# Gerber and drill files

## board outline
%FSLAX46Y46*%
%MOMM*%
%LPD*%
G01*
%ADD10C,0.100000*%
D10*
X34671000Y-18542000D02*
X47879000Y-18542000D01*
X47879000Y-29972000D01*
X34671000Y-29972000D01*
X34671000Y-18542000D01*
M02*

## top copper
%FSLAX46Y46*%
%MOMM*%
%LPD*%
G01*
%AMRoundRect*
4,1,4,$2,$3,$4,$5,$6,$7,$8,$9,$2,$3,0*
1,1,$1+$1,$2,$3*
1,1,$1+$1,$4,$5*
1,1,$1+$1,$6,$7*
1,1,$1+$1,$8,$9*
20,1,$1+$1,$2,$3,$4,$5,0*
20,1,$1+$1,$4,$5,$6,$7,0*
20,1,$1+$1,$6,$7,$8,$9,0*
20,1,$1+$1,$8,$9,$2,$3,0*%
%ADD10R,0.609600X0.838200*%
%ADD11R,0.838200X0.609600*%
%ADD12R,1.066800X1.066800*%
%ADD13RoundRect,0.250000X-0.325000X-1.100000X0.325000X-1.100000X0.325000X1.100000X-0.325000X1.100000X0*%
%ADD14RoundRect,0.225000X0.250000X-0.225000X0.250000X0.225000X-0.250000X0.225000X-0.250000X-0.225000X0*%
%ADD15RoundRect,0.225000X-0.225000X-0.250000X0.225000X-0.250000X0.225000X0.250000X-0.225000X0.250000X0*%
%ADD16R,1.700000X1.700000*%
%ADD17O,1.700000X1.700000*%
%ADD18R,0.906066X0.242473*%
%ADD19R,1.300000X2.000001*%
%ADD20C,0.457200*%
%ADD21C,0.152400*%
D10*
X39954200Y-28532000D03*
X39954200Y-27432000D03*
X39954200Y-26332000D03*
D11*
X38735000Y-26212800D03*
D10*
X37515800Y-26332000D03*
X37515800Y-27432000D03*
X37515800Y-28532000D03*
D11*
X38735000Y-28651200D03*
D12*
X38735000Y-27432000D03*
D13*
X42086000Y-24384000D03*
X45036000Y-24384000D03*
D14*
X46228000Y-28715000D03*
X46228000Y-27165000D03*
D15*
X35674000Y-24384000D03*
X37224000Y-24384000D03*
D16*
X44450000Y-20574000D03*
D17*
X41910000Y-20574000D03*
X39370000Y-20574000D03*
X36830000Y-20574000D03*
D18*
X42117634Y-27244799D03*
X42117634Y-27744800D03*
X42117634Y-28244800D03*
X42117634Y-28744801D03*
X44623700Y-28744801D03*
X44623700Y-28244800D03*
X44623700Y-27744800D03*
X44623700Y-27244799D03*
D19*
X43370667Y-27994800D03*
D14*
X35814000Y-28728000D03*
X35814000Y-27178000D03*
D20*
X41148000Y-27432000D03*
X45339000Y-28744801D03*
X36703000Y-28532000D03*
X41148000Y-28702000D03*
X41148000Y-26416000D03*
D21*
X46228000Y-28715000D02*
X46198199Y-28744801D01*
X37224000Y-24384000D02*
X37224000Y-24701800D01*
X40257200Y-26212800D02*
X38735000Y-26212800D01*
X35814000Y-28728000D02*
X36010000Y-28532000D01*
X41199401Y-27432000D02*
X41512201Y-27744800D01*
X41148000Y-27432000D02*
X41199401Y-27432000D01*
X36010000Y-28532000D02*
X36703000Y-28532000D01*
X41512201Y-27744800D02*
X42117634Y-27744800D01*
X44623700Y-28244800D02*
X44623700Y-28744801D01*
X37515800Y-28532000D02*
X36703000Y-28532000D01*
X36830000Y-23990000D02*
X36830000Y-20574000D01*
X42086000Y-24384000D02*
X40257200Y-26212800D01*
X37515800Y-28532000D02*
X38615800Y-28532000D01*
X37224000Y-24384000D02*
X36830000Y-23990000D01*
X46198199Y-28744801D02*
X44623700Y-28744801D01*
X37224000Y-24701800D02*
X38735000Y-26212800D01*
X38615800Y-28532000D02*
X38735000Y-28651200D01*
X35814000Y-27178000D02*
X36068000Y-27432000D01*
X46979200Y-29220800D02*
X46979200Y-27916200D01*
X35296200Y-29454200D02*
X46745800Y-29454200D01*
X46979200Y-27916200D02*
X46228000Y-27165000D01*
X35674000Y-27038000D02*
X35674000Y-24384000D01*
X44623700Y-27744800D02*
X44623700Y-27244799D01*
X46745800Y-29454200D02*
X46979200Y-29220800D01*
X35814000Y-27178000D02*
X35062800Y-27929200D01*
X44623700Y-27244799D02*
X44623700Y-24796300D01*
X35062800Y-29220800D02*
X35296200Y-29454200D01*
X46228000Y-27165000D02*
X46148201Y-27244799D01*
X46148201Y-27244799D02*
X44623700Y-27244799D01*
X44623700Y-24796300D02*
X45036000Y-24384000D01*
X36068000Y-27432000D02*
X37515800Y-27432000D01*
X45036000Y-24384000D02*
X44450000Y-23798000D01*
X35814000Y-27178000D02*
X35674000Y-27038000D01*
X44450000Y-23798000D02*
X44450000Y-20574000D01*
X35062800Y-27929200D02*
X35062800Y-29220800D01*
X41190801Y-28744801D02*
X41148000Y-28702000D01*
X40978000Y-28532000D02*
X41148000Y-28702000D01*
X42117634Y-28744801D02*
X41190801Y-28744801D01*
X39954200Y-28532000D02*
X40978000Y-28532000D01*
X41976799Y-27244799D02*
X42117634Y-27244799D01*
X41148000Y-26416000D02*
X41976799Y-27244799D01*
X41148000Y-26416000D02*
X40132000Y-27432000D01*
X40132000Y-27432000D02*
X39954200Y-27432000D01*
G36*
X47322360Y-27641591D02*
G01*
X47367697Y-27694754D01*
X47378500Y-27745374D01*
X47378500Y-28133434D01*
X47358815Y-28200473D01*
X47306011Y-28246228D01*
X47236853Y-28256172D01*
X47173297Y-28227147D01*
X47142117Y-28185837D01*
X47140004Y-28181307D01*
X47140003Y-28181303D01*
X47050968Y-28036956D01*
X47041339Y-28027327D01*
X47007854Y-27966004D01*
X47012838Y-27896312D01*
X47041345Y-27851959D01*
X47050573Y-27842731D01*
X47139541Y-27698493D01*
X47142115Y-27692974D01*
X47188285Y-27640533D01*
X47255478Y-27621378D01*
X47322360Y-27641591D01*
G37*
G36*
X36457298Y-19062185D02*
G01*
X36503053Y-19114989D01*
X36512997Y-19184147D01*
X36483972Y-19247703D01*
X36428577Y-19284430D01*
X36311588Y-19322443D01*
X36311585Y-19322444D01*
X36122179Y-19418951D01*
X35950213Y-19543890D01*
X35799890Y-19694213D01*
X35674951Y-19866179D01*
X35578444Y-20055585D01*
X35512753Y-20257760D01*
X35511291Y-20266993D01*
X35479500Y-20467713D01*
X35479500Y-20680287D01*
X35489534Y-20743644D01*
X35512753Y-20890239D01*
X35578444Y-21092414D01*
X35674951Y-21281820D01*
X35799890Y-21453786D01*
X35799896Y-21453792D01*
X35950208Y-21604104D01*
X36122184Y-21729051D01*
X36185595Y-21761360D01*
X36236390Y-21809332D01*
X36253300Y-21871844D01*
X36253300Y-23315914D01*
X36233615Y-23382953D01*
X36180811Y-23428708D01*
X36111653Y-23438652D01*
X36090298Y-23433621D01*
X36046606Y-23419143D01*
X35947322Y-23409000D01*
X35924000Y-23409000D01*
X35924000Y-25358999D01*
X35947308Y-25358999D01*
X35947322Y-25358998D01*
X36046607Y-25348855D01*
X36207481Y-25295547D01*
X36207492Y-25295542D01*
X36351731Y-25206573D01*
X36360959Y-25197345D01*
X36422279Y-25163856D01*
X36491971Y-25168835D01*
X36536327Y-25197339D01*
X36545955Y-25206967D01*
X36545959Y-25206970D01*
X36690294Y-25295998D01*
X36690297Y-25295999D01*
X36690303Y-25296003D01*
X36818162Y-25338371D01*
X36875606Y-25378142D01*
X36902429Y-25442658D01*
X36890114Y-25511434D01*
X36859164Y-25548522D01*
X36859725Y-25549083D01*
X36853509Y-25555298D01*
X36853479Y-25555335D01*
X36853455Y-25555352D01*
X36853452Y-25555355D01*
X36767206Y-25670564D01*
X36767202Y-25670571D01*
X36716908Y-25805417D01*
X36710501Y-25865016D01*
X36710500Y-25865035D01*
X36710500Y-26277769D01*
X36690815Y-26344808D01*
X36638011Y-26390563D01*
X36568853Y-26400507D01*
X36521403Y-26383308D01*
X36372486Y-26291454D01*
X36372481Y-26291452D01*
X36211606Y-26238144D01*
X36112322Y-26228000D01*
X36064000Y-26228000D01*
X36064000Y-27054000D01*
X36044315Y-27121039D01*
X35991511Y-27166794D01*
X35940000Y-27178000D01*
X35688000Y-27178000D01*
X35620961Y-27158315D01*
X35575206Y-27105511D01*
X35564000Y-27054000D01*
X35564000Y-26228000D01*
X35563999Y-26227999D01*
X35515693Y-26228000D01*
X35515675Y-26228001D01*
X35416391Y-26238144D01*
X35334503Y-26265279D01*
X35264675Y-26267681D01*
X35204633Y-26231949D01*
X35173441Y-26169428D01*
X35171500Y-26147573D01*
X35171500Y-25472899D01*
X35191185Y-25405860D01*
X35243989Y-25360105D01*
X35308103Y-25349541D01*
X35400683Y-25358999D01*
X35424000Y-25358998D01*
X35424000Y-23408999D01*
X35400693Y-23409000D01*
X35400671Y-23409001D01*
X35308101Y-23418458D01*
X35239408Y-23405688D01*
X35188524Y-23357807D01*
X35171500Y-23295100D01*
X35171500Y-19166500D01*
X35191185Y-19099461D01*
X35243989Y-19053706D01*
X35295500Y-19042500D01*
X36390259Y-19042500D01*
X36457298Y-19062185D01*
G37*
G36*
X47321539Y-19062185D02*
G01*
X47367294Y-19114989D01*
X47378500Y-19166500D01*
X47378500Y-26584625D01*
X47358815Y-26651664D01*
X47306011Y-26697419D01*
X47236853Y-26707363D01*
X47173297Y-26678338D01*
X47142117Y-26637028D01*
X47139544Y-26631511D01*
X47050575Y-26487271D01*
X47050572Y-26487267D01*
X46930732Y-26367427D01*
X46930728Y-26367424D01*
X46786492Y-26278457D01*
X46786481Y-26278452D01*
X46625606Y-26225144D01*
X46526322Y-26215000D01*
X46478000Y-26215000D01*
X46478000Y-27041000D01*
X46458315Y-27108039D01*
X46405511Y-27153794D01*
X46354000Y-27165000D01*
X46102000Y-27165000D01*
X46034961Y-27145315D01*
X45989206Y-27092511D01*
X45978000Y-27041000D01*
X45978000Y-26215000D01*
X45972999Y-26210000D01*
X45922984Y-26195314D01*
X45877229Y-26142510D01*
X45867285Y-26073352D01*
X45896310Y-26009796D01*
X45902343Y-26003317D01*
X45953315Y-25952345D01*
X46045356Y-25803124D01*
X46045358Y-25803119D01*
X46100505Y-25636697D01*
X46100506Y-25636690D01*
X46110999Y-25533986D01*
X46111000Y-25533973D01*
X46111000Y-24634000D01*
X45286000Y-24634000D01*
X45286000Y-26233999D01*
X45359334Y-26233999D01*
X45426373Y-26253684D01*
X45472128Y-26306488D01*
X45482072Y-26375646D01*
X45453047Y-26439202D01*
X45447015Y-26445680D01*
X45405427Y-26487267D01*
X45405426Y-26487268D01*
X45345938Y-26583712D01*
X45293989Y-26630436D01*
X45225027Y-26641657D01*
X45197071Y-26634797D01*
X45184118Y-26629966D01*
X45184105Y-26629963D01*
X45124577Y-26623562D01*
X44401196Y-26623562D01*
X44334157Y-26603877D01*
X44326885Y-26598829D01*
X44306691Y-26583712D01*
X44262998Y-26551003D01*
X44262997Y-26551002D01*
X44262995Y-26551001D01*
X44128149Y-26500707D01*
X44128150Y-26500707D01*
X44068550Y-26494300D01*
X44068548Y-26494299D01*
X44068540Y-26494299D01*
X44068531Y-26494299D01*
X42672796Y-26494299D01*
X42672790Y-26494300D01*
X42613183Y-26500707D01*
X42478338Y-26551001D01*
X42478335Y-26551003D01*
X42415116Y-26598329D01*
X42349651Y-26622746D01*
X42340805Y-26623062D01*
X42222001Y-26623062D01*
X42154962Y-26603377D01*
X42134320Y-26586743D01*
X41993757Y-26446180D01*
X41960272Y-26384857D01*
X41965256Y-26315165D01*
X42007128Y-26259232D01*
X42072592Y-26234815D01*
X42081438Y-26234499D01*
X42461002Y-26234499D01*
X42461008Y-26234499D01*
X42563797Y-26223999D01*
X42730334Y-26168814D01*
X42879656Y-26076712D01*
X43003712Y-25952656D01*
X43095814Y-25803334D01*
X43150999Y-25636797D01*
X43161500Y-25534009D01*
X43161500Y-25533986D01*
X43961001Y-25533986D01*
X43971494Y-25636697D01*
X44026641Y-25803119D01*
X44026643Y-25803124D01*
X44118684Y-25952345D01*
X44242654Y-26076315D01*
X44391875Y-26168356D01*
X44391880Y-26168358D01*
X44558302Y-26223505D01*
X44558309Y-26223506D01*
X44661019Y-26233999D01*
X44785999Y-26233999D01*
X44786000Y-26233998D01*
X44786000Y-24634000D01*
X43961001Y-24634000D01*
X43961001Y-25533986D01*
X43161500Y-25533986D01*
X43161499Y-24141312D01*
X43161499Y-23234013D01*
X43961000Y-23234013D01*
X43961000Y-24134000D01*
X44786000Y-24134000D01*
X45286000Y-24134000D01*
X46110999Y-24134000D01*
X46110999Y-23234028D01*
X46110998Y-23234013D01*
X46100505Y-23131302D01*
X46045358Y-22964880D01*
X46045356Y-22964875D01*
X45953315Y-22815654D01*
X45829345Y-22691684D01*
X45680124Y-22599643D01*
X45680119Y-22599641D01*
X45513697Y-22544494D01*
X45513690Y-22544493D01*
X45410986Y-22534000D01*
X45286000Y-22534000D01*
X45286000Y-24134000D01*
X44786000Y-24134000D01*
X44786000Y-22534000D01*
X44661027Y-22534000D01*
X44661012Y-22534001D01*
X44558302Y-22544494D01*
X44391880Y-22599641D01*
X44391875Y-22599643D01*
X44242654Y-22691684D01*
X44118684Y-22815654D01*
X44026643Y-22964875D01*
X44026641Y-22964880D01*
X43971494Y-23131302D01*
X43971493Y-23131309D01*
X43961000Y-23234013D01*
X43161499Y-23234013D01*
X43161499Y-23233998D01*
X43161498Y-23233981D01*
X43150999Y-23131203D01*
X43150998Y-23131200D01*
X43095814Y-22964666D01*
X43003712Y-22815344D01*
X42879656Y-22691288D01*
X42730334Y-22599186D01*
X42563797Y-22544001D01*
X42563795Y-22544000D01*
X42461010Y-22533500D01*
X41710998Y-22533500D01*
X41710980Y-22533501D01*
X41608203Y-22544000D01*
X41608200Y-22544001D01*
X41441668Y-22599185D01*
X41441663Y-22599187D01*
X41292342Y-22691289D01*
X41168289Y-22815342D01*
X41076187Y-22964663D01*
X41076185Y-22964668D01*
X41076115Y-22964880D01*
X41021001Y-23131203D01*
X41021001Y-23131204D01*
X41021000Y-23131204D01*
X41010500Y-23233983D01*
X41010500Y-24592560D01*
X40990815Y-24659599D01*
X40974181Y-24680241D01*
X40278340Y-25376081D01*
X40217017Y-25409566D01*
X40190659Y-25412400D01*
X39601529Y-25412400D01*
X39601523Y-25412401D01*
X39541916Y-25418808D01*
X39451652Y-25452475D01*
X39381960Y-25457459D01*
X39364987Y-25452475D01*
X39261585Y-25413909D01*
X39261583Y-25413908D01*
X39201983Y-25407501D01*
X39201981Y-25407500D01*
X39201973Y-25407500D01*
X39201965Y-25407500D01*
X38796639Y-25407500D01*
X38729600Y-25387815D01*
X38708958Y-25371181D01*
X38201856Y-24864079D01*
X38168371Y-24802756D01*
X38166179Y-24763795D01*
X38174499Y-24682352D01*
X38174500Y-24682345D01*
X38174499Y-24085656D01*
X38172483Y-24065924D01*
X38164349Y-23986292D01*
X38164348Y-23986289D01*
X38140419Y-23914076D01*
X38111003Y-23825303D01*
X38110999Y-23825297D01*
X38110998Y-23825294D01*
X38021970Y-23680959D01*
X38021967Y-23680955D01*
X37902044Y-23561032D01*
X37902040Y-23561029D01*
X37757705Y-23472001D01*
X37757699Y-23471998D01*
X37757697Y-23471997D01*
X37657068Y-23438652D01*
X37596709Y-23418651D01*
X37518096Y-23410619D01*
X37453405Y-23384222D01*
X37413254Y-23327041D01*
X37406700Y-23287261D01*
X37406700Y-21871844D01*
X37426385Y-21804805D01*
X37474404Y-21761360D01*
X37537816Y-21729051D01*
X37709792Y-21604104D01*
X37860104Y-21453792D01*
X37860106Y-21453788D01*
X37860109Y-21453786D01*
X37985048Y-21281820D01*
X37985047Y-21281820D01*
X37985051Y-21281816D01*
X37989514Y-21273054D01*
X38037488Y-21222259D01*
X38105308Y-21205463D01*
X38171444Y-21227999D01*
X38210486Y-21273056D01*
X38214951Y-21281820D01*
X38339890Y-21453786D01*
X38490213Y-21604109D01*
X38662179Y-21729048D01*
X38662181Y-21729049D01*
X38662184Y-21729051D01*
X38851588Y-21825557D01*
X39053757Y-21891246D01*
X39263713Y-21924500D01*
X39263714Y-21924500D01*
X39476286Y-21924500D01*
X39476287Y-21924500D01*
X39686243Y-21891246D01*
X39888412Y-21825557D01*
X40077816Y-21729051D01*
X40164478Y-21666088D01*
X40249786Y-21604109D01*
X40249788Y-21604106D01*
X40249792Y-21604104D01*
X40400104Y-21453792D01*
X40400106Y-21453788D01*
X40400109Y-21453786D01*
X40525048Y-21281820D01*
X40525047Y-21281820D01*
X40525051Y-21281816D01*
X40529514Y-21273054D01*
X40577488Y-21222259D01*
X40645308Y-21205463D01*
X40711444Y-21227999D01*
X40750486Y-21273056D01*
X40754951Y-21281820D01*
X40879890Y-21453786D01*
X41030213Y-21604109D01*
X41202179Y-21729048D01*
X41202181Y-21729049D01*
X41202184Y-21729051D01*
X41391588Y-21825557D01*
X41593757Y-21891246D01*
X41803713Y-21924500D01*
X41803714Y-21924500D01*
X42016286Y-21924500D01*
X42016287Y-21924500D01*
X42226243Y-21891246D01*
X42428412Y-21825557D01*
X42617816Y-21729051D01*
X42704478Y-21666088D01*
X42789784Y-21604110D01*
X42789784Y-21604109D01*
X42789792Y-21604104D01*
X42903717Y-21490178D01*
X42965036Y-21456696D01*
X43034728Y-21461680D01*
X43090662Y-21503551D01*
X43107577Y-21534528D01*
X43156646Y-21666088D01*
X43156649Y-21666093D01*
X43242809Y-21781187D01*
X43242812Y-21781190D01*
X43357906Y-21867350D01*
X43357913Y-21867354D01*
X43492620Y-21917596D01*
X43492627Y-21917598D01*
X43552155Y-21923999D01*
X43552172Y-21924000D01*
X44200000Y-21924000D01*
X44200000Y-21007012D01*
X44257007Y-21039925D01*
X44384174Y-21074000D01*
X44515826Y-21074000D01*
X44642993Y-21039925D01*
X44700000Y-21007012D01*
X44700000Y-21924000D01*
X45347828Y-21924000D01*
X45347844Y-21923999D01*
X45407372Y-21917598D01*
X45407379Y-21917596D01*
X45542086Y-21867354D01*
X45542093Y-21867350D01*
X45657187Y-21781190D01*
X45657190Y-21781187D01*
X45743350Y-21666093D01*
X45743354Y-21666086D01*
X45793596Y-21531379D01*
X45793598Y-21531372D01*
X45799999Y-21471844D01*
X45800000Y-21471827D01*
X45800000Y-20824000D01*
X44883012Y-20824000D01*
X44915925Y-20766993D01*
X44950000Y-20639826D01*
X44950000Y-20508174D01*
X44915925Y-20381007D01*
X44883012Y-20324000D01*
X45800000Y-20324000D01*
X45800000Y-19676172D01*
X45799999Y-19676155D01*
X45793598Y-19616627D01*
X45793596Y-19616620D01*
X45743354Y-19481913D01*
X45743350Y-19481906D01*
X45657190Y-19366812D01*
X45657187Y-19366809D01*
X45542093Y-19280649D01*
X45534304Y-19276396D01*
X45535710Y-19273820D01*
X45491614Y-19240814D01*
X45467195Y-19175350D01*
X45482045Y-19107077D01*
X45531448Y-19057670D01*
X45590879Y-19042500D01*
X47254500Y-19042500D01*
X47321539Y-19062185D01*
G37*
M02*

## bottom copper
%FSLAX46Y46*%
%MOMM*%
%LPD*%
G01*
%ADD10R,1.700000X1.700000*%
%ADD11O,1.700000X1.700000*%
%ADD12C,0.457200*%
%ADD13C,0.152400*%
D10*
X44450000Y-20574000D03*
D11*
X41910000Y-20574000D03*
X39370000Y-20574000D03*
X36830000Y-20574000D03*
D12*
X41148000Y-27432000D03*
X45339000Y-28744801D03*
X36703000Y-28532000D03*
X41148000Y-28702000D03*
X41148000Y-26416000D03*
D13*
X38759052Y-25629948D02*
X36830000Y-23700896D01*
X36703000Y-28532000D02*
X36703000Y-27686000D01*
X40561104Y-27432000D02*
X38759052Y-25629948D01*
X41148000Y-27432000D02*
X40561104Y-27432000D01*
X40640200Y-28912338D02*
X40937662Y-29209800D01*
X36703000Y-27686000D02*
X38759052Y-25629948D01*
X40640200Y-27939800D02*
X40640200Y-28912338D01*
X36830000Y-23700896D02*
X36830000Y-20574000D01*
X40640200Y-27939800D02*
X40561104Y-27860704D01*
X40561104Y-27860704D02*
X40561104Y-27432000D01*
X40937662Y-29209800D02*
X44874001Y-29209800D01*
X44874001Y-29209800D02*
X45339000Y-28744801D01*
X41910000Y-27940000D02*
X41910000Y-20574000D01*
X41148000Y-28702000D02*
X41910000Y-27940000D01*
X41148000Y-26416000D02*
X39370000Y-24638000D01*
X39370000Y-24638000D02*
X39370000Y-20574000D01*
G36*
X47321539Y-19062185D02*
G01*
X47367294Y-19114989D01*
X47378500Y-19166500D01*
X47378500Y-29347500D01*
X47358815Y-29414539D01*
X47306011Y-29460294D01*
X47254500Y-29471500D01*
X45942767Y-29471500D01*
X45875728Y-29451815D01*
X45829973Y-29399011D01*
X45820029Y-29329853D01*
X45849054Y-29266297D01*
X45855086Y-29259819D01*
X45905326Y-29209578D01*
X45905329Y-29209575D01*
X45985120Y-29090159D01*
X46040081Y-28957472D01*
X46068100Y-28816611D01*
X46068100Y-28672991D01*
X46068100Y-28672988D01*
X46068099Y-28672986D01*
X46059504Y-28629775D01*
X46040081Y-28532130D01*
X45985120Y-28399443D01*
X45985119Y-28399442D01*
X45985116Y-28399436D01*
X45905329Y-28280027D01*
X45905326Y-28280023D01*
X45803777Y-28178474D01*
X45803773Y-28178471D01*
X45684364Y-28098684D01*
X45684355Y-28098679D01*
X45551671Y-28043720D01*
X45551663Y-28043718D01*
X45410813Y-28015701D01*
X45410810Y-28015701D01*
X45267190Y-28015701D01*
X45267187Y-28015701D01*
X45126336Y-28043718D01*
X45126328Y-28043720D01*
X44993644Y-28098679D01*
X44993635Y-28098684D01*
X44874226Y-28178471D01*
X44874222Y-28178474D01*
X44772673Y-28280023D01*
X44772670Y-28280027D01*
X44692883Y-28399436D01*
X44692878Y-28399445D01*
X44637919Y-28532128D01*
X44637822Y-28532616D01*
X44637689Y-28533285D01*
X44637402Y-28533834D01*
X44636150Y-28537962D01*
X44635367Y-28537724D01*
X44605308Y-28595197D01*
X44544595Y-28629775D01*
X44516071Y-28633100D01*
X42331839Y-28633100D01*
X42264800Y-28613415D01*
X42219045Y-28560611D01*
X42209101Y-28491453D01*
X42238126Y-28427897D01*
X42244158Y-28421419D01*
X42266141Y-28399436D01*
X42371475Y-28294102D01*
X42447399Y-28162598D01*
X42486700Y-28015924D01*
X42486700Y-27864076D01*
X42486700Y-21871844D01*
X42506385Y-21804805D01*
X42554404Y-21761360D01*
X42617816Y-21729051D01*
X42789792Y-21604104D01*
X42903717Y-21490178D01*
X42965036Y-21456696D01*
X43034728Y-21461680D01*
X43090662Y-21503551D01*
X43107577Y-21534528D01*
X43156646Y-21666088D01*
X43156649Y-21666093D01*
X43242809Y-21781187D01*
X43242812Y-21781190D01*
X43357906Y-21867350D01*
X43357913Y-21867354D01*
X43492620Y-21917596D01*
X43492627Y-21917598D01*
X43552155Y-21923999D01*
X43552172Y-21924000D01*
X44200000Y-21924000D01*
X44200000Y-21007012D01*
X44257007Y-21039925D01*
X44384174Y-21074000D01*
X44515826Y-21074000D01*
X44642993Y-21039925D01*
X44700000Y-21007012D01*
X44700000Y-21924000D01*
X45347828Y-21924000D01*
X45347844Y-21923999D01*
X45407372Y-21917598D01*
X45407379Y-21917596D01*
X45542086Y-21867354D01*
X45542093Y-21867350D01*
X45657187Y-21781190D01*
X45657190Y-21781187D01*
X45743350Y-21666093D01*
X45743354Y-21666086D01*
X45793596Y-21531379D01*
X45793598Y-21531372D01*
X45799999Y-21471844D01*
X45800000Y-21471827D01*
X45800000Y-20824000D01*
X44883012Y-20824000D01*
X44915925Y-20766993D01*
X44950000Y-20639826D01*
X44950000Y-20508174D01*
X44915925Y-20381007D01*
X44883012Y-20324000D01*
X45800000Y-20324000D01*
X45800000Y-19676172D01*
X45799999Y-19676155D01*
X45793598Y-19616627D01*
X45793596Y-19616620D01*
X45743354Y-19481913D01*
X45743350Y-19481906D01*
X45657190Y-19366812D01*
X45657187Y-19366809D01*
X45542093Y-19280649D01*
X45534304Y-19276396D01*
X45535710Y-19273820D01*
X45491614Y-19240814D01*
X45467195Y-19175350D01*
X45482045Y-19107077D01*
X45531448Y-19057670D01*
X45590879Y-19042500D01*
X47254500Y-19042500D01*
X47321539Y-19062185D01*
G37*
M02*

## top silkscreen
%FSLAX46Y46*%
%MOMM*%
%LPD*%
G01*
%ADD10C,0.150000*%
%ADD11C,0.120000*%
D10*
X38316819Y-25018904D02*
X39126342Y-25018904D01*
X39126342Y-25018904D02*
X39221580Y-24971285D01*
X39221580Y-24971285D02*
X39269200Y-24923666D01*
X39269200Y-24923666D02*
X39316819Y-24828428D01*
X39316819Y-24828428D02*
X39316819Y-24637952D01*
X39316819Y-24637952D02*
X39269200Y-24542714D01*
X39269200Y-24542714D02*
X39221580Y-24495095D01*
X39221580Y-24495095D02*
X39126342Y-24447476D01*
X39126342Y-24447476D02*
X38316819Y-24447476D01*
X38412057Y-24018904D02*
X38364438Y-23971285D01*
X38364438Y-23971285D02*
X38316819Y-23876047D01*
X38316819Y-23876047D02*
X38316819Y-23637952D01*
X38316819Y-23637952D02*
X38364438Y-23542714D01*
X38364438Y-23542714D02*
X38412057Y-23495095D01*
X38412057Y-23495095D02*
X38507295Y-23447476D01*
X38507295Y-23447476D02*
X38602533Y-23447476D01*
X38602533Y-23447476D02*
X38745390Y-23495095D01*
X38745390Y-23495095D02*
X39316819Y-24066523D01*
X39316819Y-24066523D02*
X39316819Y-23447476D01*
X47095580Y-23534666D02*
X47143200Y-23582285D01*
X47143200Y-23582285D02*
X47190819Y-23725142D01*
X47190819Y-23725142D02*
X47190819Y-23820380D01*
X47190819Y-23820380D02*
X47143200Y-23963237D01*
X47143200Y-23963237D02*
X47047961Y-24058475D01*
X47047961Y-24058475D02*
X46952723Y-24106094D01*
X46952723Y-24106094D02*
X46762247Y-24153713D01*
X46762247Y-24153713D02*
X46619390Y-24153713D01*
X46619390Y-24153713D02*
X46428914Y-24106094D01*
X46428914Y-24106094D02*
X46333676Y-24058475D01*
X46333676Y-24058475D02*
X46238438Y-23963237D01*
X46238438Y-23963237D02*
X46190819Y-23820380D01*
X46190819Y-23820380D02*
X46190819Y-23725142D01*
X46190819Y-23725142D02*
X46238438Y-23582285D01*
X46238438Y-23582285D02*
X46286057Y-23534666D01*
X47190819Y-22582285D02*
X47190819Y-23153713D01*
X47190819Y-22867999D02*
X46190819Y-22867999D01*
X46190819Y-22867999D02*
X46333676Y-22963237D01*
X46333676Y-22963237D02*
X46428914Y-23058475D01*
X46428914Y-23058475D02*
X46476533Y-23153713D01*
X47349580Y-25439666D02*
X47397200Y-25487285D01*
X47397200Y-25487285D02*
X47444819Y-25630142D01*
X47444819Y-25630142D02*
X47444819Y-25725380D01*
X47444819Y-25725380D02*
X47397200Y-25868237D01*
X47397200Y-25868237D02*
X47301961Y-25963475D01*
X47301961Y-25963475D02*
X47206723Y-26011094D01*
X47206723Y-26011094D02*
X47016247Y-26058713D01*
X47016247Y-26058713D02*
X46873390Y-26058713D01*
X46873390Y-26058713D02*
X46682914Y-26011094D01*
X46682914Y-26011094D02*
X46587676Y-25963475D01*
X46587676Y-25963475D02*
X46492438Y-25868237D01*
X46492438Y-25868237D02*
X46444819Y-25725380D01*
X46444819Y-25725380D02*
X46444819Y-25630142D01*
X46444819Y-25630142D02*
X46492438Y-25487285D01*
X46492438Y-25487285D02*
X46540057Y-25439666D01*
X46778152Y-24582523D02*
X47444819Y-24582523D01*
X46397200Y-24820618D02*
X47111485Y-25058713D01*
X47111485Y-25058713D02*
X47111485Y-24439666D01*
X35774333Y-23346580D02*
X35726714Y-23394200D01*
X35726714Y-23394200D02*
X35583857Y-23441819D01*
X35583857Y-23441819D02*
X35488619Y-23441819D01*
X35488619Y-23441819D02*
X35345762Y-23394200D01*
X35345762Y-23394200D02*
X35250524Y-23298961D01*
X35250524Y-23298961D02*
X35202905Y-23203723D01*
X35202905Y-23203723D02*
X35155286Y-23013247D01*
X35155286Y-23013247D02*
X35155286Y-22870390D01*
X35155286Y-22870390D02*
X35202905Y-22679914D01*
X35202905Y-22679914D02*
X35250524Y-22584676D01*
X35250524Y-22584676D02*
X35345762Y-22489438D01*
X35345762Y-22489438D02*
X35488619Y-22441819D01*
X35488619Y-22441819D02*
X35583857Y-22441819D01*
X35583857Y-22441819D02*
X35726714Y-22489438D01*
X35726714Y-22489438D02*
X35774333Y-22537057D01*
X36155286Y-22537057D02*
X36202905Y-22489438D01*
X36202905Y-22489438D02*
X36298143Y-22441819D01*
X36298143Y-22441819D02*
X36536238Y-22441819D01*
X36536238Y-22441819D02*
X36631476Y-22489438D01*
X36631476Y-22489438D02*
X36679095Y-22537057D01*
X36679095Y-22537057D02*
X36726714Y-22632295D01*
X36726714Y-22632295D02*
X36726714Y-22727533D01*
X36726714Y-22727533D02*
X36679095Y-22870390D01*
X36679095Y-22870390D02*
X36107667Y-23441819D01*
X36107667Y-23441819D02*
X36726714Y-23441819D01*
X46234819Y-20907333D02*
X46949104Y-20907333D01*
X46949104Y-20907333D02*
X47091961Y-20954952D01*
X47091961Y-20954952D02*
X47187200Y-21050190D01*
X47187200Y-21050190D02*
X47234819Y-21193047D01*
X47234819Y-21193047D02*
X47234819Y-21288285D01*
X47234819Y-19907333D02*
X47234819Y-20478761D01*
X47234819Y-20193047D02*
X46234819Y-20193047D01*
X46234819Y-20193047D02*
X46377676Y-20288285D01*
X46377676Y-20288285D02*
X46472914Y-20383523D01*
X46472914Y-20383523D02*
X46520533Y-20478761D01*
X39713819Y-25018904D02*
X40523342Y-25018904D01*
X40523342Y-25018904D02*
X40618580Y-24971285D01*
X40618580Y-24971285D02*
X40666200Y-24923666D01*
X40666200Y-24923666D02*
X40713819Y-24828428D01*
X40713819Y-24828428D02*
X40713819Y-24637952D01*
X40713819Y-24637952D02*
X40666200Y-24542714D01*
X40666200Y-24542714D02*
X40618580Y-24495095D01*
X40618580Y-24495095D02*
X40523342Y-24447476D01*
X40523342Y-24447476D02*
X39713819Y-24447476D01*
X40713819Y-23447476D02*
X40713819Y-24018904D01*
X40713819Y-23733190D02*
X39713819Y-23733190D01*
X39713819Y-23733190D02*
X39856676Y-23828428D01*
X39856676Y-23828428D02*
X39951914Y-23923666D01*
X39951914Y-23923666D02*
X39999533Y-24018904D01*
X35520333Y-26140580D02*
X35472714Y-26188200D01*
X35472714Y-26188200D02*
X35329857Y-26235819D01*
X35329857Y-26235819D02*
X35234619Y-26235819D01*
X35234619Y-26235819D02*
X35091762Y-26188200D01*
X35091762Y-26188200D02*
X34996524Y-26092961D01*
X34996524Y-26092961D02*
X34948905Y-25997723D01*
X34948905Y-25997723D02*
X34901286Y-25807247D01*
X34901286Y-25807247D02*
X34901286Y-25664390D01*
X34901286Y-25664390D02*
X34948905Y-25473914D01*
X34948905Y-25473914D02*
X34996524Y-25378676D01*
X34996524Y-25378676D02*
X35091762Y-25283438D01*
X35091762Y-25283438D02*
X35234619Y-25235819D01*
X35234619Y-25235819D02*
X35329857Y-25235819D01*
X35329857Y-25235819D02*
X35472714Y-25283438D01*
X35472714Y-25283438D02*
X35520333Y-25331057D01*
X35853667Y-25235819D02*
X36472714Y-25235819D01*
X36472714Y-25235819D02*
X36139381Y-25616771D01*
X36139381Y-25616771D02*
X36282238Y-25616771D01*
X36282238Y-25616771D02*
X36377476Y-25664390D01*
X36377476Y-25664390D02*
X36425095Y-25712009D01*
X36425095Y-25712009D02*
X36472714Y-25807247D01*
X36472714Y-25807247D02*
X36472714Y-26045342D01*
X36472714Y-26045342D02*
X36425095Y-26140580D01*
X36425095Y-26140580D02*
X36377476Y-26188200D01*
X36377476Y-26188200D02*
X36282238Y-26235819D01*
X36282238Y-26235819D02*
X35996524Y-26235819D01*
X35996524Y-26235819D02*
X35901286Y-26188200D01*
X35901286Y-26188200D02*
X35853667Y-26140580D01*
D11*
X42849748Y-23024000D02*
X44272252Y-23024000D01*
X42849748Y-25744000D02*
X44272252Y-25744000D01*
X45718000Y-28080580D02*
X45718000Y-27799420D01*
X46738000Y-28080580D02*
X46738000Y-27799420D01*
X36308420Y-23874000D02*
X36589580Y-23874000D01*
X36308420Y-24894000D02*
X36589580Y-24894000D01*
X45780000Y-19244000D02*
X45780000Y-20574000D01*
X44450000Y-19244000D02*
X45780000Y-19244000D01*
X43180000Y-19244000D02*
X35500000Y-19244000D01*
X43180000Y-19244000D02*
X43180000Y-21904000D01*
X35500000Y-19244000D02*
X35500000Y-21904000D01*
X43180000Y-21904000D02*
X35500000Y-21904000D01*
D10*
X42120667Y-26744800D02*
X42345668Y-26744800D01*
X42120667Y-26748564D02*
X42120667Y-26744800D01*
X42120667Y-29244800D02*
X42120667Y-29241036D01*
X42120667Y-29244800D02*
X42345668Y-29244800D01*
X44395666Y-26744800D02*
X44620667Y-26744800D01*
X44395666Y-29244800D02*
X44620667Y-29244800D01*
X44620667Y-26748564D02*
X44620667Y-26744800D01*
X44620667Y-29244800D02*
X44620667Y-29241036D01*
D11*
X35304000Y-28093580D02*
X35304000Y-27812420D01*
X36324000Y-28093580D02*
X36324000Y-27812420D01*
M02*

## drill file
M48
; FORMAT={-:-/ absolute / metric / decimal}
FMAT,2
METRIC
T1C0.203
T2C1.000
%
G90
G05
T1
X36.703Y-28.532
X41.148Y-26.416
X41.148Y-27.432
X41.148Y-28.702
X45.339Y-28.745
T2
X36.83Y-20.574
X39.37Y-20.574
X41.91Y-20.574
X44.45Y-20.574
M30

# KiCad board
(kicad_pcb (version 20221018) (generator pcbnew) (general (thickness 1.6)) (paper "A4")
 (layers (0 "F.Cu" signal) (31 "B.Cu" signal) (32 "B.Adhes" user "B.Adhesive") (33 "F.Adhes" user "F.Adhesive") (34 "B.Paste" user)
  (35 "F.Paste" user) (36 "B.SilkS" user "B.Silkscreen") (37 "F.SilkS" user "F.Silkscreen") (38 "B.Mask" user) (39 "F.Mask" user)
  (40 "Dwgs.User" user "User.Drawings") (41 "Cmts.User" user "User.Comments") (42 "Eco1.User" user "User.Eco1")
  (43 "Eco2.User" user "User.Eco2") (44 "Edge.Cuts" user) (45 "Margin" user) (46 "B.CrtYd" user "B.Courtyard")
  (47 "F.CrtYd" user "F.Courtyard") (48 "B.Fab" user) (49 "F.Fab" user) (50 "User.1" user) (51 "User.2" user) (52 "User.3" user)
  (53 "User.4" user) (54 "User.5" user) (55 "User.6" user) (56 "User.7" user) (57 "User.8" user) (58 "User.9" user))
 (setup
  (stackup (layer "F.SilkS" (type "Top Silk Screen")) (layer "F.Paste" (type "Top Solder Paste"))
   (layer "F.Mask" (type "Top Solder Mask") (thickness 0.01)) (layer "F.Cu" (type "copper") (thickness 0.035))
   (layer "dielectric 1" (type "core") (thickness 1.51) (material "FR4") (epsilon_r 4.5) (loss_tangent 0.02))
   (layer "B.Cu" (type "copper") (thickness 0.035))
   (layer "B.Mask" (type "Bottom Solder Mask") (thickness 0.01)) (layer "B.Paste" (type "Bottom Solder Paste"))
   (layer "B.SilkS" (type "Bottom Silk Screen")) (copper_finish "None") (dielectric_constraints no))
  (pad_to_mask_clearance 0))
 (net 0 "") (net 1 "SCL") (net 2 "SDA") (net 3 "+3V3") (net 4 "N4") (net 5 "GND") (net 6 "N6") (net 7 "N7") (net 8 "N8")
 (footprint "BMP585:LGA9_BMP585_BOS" (layer "F.Cu") (at 38.735 27.432 180)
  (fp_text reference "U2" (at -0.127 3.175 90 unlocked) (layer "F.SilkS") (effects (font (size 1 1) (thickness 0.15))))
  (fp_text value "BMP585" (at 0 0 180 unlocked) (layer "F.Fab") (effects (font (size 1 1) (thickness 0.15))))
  (pad "1" smd rect (at -1.2192 -1.1 270) (size 0.8382 0.6096) (layers "F.Cu" "F.Paste" "F.Mask") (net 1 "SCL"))
  (pad "2" smd rect (at -1.2192 0 270) (size 0.8382 0.6096) (layers "F.Cu" "F.Paste" "F.Mask") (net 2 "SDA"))
  (pad "3" smd rect (at -1.2192 1.1 270) (size 0.8382 0.6096) (layers "F.Cu" "F.Paste" "F.Mask") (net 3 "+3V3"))
  (pad "4" smd rect (at 0 1.2192 180) (size 0.8382 0.6096) (layers "F.Cu" "F.Paste" "F.Mask") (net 3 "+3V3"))
  (pad "5" smd rect (at 1.2192 1.1 270) (size 0.8382 0.6096) (layers "F.Cu" "F.Paste" "F.Mask") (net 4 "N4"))
  (pad "6" smd rect (at 1.2192 0 270) (size 0.8382 0.6096) (layers "F.Cu" "F.Paste" "F.Mask") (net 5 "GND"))
  (pad "7" smd rect (at 1.2192 -1.1 270) (size 0.8382 0.6096) (layers "F.Cu" "F.Paste" "F.Mask") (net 3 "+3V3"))
  (pad "8" smd rect (at 0 -1.2192 180) (size 0.8382 0.6096) (layers "F.Cu" "F.Paste" "F.Mask") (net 3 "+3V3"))
  (pad "9" smd rect (at 0 0 180) (size 1.0668 1.0668) (layers "F.Cu" "F.Paste" "F.Mask") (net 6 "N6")))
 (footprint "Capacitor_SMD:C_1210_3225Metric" (layer "F.Cu") (at 43.561 24.384)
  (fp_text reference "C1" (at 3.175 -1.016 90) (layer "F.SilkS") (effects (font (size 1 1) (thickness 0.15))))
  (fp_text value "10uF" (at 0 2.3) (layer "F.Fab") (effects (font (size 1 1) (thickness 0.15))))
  (fp_line (start -0.711252 -1.36) (end 0.711252 -1.36) (stroke (width 0.12) (type solid)) (layer "F.SilkS"))
  (fp_line (start -0.711252 1.36) (end 0.711252 1.36) (stroke (width 0.12) (type solid)) (layer "F.SilkS"))
  (pad "1" smd roundrect (at -1.475 0) (size 1.15 2.7) (layers "F.Cu" "F.Paste" "F.Mask") (roundrect_rratio 0.2173913043) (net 3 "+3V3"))
  (pad "2" smd roundrect (at 1.475 0) (size 1.15 2.7) (layers "F.Cu" "F.Paste" "F.Mask") (roundrect_rratio 0.2173913043) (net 5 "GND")))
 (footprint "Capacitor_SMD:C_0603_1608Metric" (layer "F.Cu") (at 46.228 27.94 90)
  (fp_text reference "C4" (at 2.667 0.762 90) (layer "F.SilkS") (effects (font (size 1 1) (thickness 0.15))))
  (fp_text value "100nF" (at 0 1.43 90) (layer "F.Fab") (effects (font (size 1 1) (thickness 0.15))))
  (fp_line (start -0.14058 -0.51) (end 0.14058 -0.51) (stroke (width 0.12) (type solid)) (layer "F.SilkS"))
  (fp_line (start -0.14058 0.51) (end 0.14058 0.51) (stroke (width 0.12) (type solid)) (layer "F.SilkS"))
  (pad "1" smd roundrect (at -0.775 0 90) (size 0.9 0.95) (layers "F.Cu" "F.Paste" "F.Mask") (roundrect_rratio 0.25) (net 3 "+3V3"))
  (pad "2" smd roundrect (at 0.775 0 90) (size 0.9 0.95) (layers "F.Cu" "F.Paste" "F.Mask") (roundrect_rratio 0.25) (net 5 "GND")))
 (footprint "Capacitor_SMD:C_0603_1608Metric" (layer "F.Cu") (at 36.449 24.384)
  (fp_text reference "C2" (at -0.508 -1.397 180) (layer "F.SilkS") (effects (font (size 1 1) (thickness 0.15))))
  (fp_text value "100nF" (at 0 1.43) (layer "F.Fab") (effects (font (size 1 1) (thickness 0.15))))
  (fp_line (start -0.14058 -0.51) (end 0.14058 -0.51) (stroke (width 0.12) (type solid)) (layer "F.SilkS"))
  (fp_line (start -0.14058 0.51) (end 0.14058 0.51) (stroke (width 0.12) (type solid)) (layer "F.SilkS"))
  (pad "1" smd roundrect (at -0.775 0) (size 0.9 0.95) (layers "F.Cu" "F.Paste" "F.Mask") (roundrect_rratio 0.25) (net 5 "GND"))
  (pad "2" smd roundrect (at 0.775 0) (size 0.9 0.95) (layers "F.Cu" "F.Paste" "F.Mask") (roundrect_rratio 0.25) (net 3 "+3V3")))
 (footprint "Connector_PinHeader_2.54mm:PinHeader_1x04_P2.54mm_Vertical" (layer "F.Cu") (at 44.45 20.574 -90)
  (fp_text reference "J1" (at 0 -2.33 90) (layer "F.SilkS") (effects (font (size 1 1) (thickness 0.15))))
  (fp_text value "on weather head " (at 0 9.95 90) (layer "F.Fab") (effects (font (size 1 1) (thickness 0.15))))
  (fp_line (start -1.33 -1.33) (end 0 -1.33) (stroke (width 0.12) (type solid)) (layer "F.SilkS"))
  (fp_line (start -1.33 0) (end -1.33 -1.33) (stroke (width 0.12) (type solid)) (layer "F.SilkS"))
  (fp_line (start -1.33 1.27) (end -1.33 8.95) (stroke (width 0.12) (type solid)) (layer "F.SilkS"))
  (fp_line (start -1.33 1.27) (end 1.33 1.27) (stroke (width 0.12) (type solid)) (layer "F.SilkS"))
  (fp_line (start -1.33 8.95) (end 1.33 8.95) (stroke (width 0.12) (type solid)) (layer "F.SilkS"))
  (fp_line (start 1.33 1.27) (end 1.33 8.95) (stroke (width 0.12) (type solid)) (layer "F.SilkS"))
  (pad "1" thru_hole rect (at 0 0 270) (size 1.7 1.7) (drill 1) (layers "*.Cu" "*.Mask") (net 5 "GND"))
  (pad "2" thru_hole oval (at 0 2.54 270) (size 1.7 1.7) (drill 1) (layers "*.Cu" "*.Mask") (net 1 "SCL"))
  (pad "3" thru_hole oval (at 0 5.08 270) (size 1.7 1.7) (drill 1) (layers "*.Cu" "*.Mask") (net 2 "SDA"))
  (pad "4" thru_hole oval (at 0 7.62 270) (size 1.7 1.7) (drill 1) (layers "*.Cu" "*.Mask") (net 3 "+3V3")))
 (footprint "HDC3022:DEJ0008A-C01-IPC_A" (layer "F.Cu") (at 43.370667 27.9948)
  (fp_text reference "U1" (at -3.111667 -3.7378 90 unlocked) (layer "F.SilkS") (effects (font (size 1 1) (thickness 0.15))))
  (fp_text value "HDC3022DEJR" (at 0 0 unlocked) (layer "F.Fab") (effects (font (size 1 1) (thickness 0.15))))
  (fp_line (start -1.25 -1.25) (end -1.024999 -1.25) (stroke (width 0.15) (type solid)) (layer "F.SilkS"))
  (fp_line (start -1.25 -1.246236) (end -1.25 -1.25) (stroke (width 0.15) (type solid)) (layer "F.SilkS"))
  (fp_line (start -1.25 1.25) (end -1.25 1.246236) (stroke (width 0.15) (type solid)) (layer "F.SilkS"))
  (fp_line (start -1.25 1.25) (end -1.024999 1.25) (stroke (width 0.15) (type solid)) (layer "F.SilkS"))
  (fp_line (start 1.024999 -1.25) (end 1.25 -1.25) (stroke (width 0.15) (type solid)) (layer "F.SilkS"))
  (fp_line (start 1.024999 1.25) (end 1.25 1.25) (stroke (width 0.15) (type solid)) (layer "F.SilkS"))
  (fp_line (start 1.25 -1.246236) (end 1.25 -1.25) (stroke (width 0.15) (type solid)) (layer "F.SilkS"))
  (fp_line (start 1.25 1.25) (end 1.25 1.246236) (stroke (width 0.15) (type solid)) (layer "F.SilkS"))
  (pad "1" smd rect (at -1.253033 -0.750001) (size 0.906066 0.242473) (layers "F.Cu" "F.Paste" "F.Mask") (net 2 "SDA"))
  (pad "2" smd rect (at -1.253033 -0.25) (size 0.906066 0.242473) (layers "F.Cu" "F.Paste" "F.Mask") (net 3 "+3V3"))
  (pad "3" smd rect (at -1.253033 0.25) (size 0.906066 0.242473) (layers "F.Cu" "F.Paste" "F.Mask") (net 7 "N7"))
  (pad "4" smd rect (at -1.253033 0.750001) (size 0.906066 0.242473) (layers "F.Cu" "F.Paste" "F.Mask") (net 1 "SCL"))
  (pad "5" smd rect (at 1.253033 0.750001) (size 0.906066 0.242473) (layers "F.Cu" "F.Paste" "F.Mask") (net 3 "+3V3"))
  (pad "6" smd rect (at 1.253033 0.25) (size 0.906066 0.242473) (layers "F.Cu" "F.Paste" "F.Mask") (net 3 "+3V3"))
  (pad "7" smd rect (at 1.253033 -0.25) (size 0.906066 0.242473) (layers "F.Cu" "F.Paste" "F.Mask") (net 5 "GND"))
  (pad "8" smd rect (at 1.253033 -0.750001) (size 0.906066 0.242473) (layers "F.Cu" "F.Paste" "F.Mask") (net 5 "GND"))
  (pad "9" smd rect (at 0 0) (size 1.3 2.000001) (layers "F.Cu" "F.Mask") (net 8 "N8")))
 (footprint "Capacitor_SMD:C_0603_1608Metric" (layer "F.Cu") (at 35.814 27.953 90)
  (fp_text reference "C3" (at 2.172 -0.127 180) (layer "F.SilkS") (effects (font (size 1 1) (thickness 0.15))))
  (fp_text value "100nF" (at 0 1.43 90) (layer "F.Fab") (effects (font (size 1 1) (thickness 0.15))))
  (fp_line (start -0.14058 -0.51) (end 0.14058 -0.51) (stroke (width 0.12) (type solid)) (layer "F.SilkS"))
  (fp_line (start -0.14058 0.51) (end 0.14058 0.51) (stroke (width 0.12) (type solid)) (layer "F.SilkS"))
  (pad "1" smd roundrect (at -0.775 0 90) (size 0.9 0.95) (layers "F.Cu" "F.Paste" "F.Mask") (roundrect_rratio 0.25) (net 3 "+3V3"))
  (pad "2" smd roundrect (at 0.775 0 90) (size 0.9 0.95) (layers "F.Cu" "F.Paste" "F.Mask") (roundrect_rratio 0.25) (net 5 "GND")))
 (gr_rect (start 34.671 18.542) (end 47.879 29.972) (stroke (width 0.1) (type default)) (fill none) (layer "Edge.Cuts"))
 (segment (start 46.228 28.715) (end 46.198199 28.744801) (width 0.1524) (layer "F.Cu") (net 3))
 (segment (start 37.224 24.384) (end 37.224 24.7018) (width 0.1524) (layer "F.Cu") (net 3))
 (segment (start 40.2572 26.2128) (end 38.735 26.2128) (width 0.1524) (layer "F.Cu") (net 3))
 (segment (start 35.814 28.728) (end 36.01 28.532) (width 0.1524) (layer "F.Cu") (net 3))
 (segment (start 41.199401 27.432) (end 41.512201 27.7448) (width 0.1524) (layer "F.Cu") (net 3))
 (segment (start 41.148 27.432) (end 41.199401 27.432) (width 0.1524) (layer "F.Cu") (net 3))
 (segment (start 36.01 28.532) (end 36.703 28.532) (width 0.1524) (layer "F.Cu") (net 3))
 (segment (start 41.512201 27.7448) (end 42.117634 27.7448) (width 0.1524) (layer "F.Cu") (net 3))
 (segment (start 44.6237 28.2448) (end 44.6237 28.744801) (width 0.1524) (layer "F.Cu") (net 3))
 (segment (start 37.5158 28.532) (end 36.703 28.532) (width 0.1524) (layer "F.Cu") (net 3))
 (segment (start 36.83 23.99) (end 36.83 20.574) (width 0.1524) (layer "F.Cu") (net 3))
 (segment (start 42.086 24.384) (end 40.2572 26.2128) (width 0.1524) (layer "F.Cu") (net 3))
 (segment (start 37.5158 28.532) (end 38.6158 28.532) (width 0.1524) (layer "F.Cu") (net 3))
 (segment (start 37.224 24.384) (end 36.83 23.99) (width 0.1524) (layer "F.Cu") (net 3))
 (segment (start 46.198199 28.744801) (end 44.6237 28.744801) (width 0.1524) (layer "F.Cu") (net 3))
 (segment (start 37.224 24.7018) (end 38.735 26.2128) (width 0.1524) (layer "F.Cu") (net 3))
 (segment (start 38.6158 28.532) (end 38.735 28.6512) (width 0.1524) (layer "F.Cu") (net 3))
 (via (at 41.148 27.432) (size 0.4572) (drill 0.2032) (layers "F.Cu" "B.Cu") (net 3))
 (via (at 45.339 28.744801) (size 0.4572) (drill 0.2032) (layers "F.Cu" "B.Cu") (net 3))
 (via (at 36.703 28.532) (size 0.4572) (drill 0.2032) (layers "F.Cu" "B.Cu") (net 3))
 (segment (start 38.759052 25.629948) (end 36.83 23.700896) (width 0.1524) (layer "B.Cu") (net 3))
 (segment (start 36.703 28.532) (end 36.703 27.686) (width 0.1524) (layer "B.Cu") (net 3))
 (segment (start 40.561104 27.432) (end 38.759052 25.629948) (width 0.1524) (layer "B.Cu") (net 3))
 (segment (start 41.148 27.432) (end 40.561104 27.432) (width 0.1524) (layer "B.Cu") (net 3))
 (segment (start 40.6402 28.912338) (end 40.937662 29.2098) (width 0.1524) (layer "B.Cu") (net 3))
 (segment (start 36.703 27.686) (end 38.759052 25.629948) (width 0.1524) (layer "B.Cu") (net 3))
 (segment (start 40.6402 27.9398) (end 40.6402 28.912338) (width 0.1524) (layer "B.Cu") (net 3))
 (segment (start 36.83 23.700896) (end 36.83 20.574) (width 0.1524) (layer "B.Cu") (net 3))
 (segment (start 40.6402 27.9398) (end 40.561104 27.860704) (width 0.1524) (layer "B.Cu") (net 3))
 (segment (start 40.561104 27.860704) (end 40.561104 27.432) (width 0.1524) (layer "B.Cu") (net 3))
 (segment (start 40.937662 29.2098) (end 44.874001 29.2098) (width 0.1524) (layer "B.Cu") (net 3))
 (segment (start 44.874001 29.2098) (end 45.339 28.744801) (width 0.1524) (layer "B.Cu") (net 3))
 (segment (start 35.814 27.178) (end 36.068 27.432) (width 0.1524) (layer "F.Cu") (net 5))
 (segment (start 46.9792 29.2208) (end 46.9792 27.9162) (width 0.1524) (layer "F.Cu") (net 5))
 (segment (start 35.2962 29.4542) (end 46.7458 29.4542) (width 0.1524) (layer "F.Cu") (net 5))
 (segment (start 46.9792 27.9162) (end 46.228 27.165) (width 0.1524) (layer "F.Cu") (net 5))
 (segment (start 35.674 27.038) (end 35.674 24.384) (width 0.1524) (layer "F.Cu") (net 5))
 (segment (start 44.6237 27.7448) (end 44.6237 27.244799) (width 0.1524) (layer "F.Cu") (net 5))
 (segment (start 46.7458 29.4542) (end 46.9792 29.2208) (width 0.1524) (layer "F.Cu") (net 5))
 (segment (start 35.814 27.178) (end 35.0628 27.9292) (width 0.1524) (layer "F.Cu") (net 5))
 (segment (start 44.6237 27.244799) (end 44.6237 24.7963) (width 0.1524) (layer "F.Cu") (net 5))
 (segment (start 35.0628 29.2208) (end 35.2962 29.4542) (width 0.1524) (layer "F.Cu") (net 5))
 (segment (start 46.228 27.165) (end 46.148201 27.244799) (width 0.1524) (layer "F.Cu") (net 5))
 (segment (start 46.148201 27.244799) (end 44.6237 27.244799) (width 0.1524) (layer "F.Cu") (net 5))
 (segment (start 44.6237 24.7963) (end 45.036 24.384) (width 0.1524) (layer "F.Cu") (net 5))
 (segment (start 36.068 27.432) (end 37.5158 27.432) (width 0.1524) (layer "F.Cu") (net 5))
 (segment (start 45.036 24.384) (end 44.45 23.798) (width 0.1524) (layer "F.Cu") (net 5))
 (segment (start 35.814 27.178) (end 35.674 27.038) (width 0.1524) (layer "F.Cu") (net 5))
 (segment (start 44.45 23.798) (end 44.45 20.574) (width 0.1524) (layer "F.Cu") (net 5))
 (segment (start 35.0628 27.9292) (end 35.0628 29.2208) (width 0.1524) (layer "F.Cu") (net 5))
 (segment (start 41.190801 28.744801) (end 41.148 28.702) (width 0.1524) (layer "F.Cu") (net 1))
 (segment (start 40.978 28.532) (end 41.148 28.702) (width 0.1524) (layer "F.Cu") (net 1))
 (segment (start 42.117634 28.744801) (end 41.190801 28.744801) (width 0.1524) (layer "F.Cu") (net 1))
 (segment (start 39.9542 28.532) (end 40.978 28.532) (width 0.1524) (layer "F.Cu") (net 1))
 (via (at 41.148 28.702) (size 0.4572) (drill 0.2032) (layers "F.Cu" "B.Cu") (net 1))
 (segment (start 41.91 27.94) (end 41.91 20.574) (width 0.1524) (layer "B.Cu") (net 1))
 (segment (start 41.148 28.702) (end 41.91 27.94) (width 0.1524) (layer "B.Cu") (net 1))
 (segment (start 41.976799 27.244799) (end 42.117634 27.244799) (width 0.1524) (layer "F.Cu") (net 2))
 (segment (start 41.148 26.416) (end 41.976799 27.244799) (width 0.1524) (layer "F.Cu") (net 2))
 (segment (start 41.148 26.416) (end 40.132 27.432) (width 0.1524) (layer "F.Cu") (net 2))
 (segment (start 40.132 27.432) (end 39.9542 27.432) (width 0.1524) (layer "F.Cu") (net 2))
 (via (at 41.148 26.416) (size 0.4572) (drill 0.2032) (layers "F.Cu" "B.Cu") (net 2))
 (segment (start 41.148 26.416) (end 39.37 24.638) (width 0.1524) (layer "B.Cu") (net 2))
 (segment (start 39.37 24.638) (end 39.37 20.574) (width 0.1524) (layer "B.Cu") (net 2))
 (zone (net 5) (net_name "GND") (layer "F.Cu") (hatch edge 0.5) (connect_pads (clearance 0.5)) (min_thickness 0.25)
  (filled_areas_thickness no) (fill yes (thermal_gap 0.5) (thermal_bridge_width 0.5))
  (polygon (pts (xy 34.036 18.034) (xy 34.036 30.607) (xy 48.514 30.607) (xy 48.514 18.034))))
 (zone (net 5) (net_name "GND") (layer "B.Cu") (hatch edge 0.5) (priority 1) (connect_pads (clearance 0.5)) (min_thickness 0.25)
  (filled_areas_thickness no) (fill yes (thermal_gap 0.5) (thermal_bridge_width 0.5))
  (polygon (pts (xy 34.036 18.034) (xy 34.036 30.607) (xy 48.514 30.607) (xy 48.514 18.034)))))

